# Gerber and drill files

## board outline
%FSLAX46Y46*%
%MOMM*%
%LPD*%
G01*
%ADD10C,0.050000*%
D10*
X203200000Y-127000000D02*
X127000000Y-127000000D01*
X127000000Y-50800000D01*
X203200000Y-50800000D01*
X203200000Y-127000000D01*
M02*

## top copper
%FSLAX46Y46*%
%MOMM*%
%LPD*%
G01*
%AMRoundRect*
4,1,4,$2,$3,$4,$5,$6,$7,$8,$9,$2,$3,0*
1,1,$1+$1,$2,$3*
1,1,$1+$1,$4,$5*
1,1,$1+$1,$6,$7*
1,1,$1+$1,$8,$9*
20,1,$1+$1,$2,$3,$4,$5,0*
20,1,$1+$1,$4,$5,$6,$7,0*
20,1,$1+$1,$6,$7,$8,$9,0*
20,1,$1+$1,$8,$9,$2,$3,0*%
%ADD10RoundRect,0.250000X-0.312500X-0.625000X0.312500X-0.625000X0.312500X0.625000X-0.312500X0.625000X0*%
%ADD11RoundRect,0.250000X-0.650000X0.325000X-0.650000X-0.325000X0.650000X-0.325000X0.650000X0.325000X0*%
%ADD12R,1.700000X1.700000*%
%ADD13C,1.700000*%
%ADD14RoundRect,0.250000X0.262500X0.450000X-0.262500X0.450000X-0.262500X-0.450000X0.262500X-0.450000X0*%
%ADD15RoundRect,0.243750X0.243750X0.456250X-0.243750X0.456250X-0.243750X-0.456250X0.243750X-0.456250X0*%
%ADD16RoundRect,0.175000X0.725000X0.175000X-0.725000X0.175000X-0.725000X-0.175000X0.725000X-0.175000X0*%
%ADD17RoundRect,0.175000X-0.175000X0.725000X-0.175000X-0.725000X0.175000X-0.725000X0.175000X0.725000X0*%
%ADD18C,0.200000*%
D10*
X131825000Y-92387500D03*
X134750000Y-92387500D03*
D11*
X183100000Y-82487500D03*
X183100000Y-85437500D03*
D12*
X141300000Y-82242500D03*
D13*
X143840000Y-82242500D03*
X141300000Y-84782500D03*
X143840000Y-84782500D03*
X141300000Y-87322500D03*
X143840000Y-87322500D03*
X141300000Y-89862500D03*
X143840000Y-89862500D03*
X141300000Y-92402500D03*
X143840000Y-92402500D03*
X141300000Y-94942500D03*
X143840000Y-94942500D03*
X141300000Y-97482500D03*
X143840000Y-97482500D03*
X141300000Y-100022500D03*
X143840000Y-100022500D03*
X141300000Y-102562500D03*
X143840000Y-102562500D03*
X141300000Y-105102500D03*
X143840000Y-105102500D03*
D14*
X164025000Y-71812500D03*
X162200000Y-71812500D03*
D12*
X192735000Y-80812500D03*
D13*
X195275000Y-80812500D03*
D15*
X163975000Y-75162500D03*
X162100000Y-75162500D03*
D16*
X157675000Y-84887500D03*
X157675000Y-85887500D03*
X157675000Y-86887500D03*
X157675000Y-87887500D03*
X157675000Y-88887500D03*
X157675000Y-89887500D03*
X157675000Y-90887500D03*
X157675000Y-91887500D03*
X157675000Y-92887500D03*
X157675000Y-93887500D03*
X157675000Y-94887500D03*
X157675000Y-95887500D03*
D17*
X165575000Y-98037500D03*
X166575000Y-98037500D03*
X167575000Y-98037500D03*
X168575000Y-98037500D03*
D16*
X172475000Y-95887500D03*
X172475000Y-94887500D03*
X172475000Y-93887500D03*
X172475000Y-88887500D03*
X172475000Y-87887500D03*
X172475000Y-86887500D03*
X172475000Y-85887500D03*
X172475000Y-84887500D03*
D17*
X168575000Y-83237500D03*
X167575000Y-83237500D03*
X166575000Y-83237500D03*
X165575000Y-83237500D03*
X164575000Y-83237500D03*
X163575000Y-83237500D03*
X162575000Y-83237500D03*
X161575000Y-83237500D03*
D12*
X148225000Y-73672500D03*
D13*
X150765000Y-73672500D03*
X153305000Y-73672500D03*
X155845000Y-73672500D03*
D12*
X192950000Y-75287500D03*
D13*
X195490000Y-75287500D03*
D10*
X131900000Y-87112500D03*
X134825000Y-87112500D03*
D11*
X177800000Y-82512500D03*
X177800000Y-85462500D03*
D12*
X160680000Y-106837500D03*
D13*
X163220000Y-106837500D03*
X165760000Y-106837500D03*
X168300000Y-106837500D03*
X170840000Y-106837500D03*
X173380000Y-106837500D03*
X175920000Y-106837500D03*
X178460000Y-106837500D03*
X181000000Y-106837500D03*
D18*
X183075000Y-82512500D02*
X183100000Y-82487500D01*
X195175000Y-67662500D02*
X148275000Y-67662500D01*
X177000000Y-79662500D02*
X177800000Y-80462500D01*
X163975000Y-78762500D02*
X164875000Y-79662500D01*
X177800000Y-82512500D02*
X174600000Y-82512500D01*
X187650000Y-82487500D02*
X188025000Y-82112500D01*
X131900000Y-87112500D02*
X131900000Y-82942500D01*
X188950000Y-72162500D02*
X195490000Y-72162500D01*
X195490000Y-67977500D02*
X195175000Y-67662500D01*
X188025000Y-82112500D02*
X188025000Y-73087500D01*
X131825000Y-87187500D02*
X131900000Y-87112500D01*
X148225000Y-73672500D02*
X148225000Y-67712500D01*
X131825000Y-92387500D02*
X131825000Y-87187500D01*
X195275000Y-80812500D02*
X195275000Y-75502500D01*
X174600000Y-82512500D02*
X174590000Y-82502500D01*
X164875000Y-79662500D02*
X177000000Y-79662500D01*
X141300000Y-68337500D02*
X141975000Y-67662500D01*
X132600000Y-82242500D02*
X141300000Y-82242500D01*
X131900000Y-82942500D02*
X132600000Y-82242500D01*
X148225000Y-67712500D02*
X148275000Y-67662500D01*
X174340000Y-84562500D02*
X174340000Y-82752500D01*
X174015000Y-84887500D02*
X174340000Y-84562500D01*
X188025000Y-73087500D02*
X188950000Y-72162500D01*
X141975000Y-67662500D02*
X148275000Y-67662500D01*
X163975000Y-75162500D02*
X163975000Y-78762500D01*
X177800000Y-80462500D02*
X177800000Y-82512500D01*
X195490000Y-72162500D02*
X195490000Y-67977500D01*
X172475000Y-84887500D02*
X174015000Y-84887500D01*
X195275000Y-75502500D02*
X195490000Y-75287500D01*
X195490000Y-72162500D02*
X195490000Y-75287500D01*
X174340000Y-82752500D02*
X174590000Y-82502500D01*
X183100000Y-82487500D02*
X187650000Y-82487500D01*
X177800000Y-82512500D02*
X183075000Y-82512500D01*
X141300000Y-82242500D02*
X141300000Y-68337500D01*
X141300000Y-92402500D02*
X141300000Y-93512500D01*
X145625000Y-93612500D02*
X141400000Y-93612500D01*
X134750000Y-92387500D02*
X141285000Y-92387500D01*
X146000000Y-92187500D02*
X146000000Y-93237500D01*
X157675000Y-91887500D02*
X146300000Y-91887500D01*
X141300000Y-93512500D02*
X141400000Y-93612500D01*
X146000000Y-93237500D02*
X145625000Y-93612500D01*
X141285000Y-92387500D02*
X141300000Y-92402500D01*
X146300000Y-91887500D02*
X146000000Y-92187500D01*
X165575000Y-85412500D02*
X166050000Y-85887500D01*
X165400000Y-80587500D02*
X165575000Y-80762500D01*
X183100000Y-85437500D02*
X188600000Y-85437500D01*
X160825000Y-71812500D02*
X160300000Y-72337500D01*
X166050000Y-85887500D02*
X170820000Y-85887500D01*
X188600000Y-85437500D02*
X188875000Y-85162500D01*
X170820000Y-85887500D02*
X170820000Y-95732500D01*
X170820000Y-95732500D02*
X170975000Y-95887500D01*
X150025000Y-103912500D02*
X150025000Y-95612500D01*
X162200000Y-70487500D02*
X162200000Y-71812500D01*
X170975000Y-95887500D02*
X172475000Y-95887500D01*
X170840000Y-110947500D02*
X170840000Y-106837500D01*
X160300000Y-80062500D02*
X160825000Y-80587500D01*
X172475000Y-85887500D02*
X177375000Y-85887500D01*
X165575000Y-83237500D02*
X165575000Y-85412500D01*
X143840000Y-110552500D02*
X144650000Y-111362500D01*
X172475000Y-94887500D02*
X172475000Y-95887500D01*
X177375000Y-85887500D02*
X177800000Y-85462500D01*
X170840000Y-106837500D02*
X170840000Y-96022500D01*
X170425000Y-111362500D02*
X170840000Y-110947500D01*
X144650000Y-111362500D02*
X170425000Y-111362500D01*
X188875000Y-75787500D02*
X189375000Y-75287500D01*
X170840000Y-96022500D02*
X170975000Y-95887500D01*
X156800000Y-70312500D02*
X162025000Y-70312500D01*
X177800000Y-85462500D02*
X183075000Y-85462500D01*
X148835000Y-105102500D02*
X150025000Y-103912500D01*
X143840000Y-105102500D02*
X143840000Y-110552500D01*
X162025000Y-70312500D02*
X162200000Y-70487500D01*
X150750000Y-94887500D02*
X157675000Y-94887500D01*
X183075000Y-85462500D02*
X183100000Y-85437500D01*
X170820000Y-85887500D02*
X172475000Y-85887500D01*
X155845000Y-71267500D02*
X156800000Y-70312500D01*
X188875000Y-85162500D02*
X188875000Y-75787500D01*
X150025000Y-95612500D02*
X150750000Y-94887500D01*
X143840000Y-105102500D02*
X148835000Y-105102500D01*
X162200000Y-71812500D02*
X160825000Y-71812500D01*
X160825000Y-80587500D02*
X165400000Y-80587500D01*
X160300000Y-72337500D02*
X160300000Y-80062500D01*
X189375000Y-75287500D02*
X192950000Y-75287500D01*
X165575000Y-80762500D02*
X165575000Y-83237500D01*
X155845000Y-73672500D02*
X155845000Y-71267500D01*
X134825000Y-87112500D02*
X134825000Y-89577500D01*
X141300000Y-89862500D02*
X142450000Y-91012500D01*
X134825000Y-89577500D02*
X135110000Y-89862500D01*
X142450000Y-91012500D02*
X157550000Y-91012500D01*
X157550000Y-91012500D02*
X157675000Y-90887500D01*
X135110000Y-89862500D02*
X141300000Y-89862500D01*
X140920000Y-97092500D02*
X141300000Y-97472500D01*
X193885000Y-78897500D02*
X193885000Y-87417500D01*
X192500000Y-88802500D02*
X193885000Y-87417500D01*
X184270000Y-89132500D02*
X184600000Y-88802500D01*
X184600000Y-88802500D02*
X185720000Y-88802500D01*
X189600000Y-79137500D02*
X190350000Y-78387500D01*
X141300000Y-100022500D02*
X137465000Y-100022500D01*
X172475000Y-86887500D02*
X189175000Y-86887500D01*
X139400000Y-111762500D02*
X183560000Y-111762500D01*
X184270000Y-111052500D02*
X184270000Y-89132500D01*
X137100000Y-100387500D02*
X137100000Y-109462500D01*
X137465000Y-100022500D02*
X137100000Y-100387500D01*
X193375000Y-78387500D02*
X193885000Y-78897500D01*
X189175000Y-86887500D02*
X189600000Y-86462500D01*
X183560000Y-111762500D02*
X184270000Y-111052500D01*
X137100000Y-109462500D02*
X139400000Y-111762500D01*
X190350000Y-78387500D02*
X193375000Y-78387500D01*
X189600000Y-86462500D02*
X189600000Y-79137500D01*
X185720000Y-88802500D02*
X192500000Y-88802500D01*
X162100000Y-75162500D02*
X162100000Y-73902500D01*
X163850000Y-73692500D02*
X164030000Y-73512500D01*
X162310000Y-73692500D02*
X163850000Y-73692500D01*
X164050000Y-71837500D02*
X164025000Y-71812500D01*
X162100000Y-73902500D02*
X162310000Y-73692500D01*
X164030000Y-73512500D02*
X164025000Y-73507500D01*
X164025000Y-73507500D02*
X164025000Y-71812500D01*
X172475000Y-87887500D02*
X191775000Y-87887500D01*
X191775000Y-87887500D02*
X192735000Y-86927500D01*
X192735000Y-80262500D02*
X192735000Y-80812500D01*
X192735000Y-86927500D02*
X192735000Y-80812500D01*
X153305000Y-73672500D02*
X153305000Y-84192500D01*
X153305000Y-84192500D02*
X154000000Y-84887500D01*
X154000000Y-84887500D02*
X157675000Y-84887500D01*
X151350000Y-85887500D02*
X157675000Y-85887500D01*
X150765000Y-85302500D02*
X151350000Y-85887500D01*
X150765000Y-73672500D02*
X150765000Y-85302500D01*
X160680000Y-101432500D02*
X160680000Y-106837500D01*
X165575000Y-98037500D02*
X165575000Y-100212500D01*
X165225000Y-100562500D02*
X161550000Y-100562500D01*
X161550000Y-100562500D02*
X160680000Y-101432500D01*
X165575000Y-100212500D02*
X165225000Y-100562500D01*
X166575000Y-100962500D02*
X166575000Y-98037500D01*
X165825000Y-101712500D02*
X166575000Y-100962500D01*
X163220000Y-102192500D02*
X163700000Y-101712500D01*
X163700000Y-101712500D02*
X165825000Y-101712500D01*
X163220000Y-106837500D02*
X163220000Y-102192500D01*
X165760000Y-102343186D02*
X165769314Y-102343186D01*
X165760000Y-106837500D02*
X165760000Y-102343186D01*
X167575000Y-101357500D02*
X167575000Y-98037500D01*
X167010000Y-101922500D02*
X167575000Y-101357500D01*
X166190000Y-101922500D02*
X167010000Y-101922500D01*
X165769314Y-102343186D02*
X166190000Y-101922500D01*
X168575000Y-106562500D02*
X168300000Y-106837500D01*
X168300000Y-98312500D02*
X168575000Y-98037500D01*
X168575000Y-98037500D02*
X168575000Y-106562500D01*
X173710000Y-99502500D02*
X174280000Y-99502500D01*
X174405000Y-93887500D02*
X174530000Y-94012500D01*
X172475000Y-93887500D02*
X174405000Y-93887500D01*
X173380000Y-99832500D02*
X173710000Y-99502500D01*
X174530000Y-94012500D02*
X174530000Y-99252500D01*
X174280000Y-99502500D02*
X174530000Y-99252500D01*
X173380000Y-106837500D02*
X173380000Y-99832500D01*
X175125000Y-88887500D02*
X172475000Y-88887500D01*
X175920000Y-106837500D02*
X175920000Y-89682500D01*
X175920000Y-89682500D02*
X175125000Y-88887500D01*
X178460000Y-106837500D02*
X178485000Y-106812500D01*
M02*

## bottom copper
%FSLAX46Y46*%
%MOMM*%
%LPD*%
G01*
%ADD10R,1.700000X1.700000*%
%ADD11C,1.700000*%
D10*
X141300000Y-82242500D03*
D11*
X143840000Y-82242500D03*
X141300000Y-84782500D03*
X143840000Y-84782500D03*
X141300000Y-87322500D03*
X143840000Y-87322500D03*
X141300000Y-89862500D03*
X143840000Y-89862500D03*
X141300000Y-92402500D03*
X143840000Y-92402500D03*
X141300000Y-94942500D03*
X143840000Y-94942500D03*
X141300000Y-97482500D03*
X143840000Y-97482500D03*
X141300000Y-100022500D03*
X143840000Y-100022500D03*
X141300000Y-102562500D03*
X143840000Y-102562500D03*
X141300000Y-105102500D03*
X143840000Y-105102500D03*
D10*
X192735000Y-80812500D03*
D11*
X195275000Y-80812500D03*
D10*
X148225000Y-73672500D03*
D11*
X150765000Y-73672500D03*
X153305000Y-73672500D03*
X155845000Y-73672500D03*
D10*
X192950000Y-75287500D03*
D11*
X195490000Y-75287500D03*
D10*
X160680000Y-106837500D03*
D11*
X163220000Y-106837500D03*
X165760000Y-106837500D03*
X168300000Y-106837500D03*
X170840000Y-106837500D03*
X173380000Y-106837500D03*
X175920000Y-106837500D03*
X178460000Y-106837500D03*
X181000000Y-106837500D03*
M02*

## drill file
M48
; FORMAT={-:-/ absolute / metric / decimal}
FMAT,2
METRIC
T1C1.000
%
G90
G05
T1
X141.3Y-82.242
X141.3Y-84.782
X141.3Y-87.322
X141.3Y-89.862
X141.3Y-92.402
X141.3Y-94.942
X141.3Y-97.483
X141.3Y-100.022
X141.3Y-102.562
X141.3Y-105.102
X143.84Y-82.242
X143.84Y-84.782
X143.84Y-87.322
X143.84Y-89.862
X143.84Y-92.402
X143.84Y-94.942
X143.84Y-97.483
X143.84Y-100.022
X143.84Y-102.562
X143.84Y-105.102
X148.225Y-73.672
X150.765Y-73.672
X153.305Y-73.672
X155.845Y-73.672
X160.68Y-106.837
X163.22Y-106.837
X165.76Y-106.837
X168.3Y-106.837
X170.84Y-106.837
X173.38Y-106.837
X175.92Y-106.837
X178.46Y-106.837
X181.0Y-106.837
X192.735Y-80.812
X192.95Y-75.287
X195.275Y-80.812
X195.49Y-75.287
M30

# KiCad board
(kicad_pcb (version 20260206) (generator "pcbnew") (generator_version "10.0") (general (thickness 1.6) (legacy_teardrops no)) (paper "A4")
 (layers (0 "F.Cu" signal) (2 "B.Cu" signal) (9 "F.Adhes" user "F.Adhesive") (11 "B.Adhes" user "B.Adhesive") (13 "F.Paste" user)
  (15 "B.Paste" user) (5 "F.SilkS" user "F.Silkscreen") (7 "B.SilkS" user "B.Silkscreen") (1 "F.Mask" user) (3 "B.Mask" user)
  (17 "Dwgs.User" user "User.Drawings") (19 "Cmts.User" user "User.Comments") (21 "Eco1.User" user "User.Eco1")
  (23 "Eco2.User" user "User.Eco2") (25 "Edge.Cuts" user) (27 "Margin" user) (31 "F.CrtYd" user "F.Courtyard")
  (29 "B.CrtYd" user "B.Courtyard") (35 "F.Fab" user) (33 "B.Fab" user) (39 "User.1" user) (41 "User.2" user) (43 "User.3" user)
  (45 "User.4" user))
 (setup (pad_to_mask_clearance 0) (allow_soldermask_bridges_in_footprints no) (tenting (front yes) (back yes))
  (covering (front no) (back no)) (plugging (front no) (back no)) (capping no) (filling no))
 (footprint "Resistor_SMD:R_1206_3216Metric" (layer "F.Cu") (at 133.2875 92.3875)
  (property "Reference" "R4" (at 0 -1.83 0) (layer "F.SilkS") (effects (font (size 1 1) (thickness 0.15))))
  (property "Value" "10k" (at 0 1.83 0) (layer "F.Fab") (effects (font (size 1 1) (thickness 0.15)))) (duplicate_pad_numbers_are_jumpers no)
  (pad "1" smd roundrect (at -1.4625 0) (size 1.125 1.75) (layers "F.Cu" "F.Mask" "F.Paste") (roundrect_rratio 0.222222) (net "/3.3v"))
  (pad "2" smd roundrect (at 1.4625 0) (size 1.125 1.75) (layers "F.Cu" "F.Mask" "F.Paste") (roundrect_rratio 0.222222) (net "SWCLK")))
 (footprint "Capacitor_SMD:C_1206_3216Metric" (layer "F.Cu") (at 183.1 83.9625 -90)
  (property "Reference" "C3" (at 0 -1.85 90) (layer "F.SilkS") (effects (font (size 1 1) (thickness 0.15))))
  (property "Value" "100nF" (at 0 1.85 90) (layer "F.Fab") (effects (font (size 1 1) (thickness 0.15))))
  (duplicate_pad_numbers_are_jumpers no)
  (pad "1" smd roundrect (at -1.475 0 270) (size 1.15 1.8) (layers "F.Cu" "F.Mask" "F.Paste") (roundrect_rratio 0.217391) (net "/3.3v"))
  (pad "2" smd roundrect (at 1.475 0 270) (size 1.15 1.8) (layers "F.Cu" "F.Mask" "F.Paste") (roundrect_rratio 0.217391) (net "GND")))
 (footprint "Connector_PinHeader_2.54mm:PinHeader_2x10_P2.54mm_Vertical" (layer "F.Cu") (at 141.3 82.2425)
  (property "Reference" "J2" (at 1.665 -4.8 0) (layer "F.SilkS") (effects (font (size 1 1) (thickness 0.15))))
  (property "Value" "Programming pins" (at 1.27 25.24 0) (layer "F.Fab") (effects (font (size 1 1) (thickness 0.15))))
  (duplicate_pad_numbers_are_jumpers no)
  (pad "1" thru_hole rect (at 0 0) (size 1.7 1.7) (drill 1) (layers "*.Cu" "*.Mask") (remove_unused_layers no) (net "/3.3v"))
  (pad "2" thru_hole circle (at 2.54 0) (size 1.7 1.7) (drill 1) (layers "*.Cu" "*.Mask") (remove_unused_layers no)
   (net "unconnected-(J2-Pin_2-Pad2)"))
  (pad "3" thru_hole circle (at 0 2.54) (size 1.7 1.7) (drill 1) (layers "*.Cu" "*.Mask") (remove_unused_layers no)
   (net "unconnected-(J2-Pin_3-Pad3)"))
  (pad "4" thru_hole circle (at 2.54 2.54) (size 1.7 1.7) (drill 1) (layers "*.Cu" "*.Mask") (remove_unused_layers no)
   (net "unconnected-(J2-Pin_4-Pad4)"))
  (pad "5" thru_hole circle (at 0 5.08) (size 1.7 1.7) (drill 1) (layers "*.Cu" "*.Mask") (remove_unused_layers no)
   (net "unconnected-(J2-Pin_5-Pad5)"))
  (pad "6" thru_hole circle (at 2.54 5.08) (size 1.7 1.7) (drill 1) (layers "*.Cu" "*.Mask") (remove_unused_layers no)
   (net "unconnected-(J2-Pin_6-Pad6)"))
  (pad "7" thru_hole circle (at 0 7.62) (size 1.7 1.7) (drill 1) (layers "*.Cu" "*.Mask") (remove_unused_layers no) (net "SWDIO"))
  (pad "8" thru_hole circle (at 2.54 7.62) (size 1.7 1.7) (drill 1) (layers "*.Cu" "*.Mask") (remove_unused_layers no)
   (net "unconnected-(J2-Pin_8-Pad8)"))
  (pad "9" thru_hole circle (at 0 10.16) (size 1.7 1.7) (drill 1) (layers "*.Cu" "*.Mask") (remove_unused_layers no) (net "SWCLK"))
  (pad "10" thru_hole circle (at 2.54 10.16) (size 1.7 1.7) (drill 1) (layers "*.Cu" "*.Mask") (remove_unused_layers no)
   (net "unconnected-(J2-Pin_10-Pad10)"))
  (pad "11" thru_hole circle (at 0 12.7) (size 1.7 1.7) (drill 1) (layers "*.Cu" "*.Mask") (remove_unused_layers no)
   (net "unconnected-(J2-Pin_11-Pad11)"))
  (pad "12" thru_hole circle (at 2.54 12.7) (size 1.7 1.7) (drill 1) (layers "*.Cu" "*.Mask") (remove_unused_layers no)
   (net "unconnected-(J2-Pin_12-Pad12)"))
  (pad "13" thru_hole circle (at 0 15.24) (size 1.7 1.7) (drill 1) (layers "*.Cu" "*.Mask") (remove_unused_layers no)
   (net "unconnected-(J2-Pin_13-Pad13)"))
  (pad "14" thru_hole circle (at 2.54 15.24) (size 1.7 1.7) (drill 1) (layers "*.Cu" "*.Mask") (remove_unused_layers no)
   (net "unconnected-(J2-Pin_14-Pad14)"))
  (pad "15" thru_hole circle (at 0 17.78) (size 1.7 1.7) (drill 1) (layers "*.Cu" "*.Mask") (remove_unused_layers no) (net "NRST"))
  (pad "16" thru_hole circle (at 2.54 17.78) (size 1.7 1.7) (drill 1) (layers "*.Cu" "*.Mask") (remove_unused_layers no)
   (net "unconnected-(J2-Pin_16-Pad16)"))
  (pad "17" thru_hole circle (at 0 20.32) (size 1.7 1.7) (drill 1) (layers "*.Cu" "*.Mask") (remove_unused_layers no)
   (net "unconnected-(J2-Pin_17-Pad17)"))
  (pad "18" thru_hole circle (at 2.54 20.32) (size 1.7 1.7) (drill 1) (layers "*.Cu" "*.Mask") (remove_unused_layers no)
   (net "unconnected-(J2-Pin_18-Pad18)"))
  (pad "19" thru_hole circle (at 0 22.86) (size 1.7 1.7) (drill 1) (layers "*.Cu" "*.Mask") (remove_unused_layers no)
   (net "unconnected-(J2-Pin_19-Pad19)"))
  (pad "20" thru_hole circle (at 2.54 22.86) (size 1.7 1.7) (drill 1) (layers "*.Cu" "*.Mask") (remove_unused_layers no) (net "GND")))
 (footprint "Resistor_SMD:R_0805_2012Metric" (layer "F.Cu") (at 163.1125 71.8125 180)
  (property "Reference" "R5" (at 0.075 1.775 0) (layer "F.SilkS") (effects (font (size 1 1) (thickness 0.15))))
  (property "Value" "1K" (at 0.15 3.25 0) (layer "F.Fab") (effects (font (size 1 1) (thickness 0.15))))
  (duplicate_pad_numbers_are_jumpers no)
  (pad "1" smd roundrect (at -0.9125 0 180) (size 1.025 1.4) (layers "F.Cu" "F.Mask" "F.Paste") (roundrect_rratio 0.243902)
   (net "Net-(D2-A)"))
  (pad "2" smd roundrect (at 0.9125 0 180) (size 1.025 1.4) (layers "F.Cu" "F.Mask" "F.Paste") (roundrect_rratio 0.243902) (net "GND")))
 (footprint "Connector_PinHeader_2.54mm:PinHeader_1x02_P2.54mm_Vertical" (layer "F.Cu") (at 192.735 80.8125 90)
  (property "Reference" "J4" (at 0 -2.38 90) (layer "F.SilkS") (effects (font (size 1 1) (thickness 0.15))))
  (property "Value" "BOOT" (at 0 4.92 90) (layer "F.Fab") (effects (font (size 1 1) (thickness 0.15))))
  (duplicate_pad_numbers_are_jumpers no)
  (pad "1" thru_hole rect (at 0 0 90) (size 1.7 1.7) (drill 1) (layers "*.Cu" "*.Mask") (remove_unused_layers no) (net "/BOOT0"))
  (pad "2" thru_hole circle (at 0 2.54 90) (size 1.7 1.7) (drill 1) (layers "*.Cu" "*.Mask") (remove_unused_layers no) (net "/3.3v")))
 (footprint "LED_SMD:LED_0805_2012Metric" (layer "F.Cu") (at 163.0375 75.1625 180)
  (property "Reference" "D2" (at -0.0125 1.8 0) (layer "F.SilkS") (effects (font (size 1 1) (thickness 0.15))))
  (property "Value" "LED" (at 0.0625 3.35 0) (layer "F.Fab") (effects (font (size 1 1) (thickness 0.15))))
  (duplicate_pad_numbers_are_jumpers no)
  (pad "1" smd roundrect (at -0.9375 0 180) (size 0.975 1.4) (layers "F.Cu" "F.Mask" "F.Paste") (roundrect_rratio 0.25) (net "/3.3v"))
  (pad "2" smd roundrect (at 0.9375 0 180) (size 0.975 1.4) (layers "F.Cu" "F.Mask" "F.Paste") (roundrect_rratio 0.25) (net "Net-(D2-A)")))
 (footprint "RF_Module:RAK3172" (layer "F.Cu") (at 165.075 90.6375)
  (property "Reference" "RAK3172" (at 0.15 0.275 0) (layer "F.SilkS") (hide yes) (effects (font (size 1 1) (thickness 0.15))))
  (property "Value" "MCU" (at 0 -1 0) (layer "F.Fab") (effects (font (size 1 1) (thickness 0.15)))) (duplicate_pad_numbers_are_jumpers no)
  (pad "1" smd roundrect (at -7.4 -5.75 180) (size 1.8 0.7) (layers "F.Cu" "F.Mask" "F.Paste") (roundrect_rratio 0.25) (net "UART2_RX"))
  (pad "2" smd roundrect (at -7.4 -4.75 180) (size 1.8 0.7) (layers "F.Cu" "F.Mask" "F.Paste") (roundrect_rratio 0.25) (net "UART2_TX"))
  (pad "3" smd roundrect (at -7.4 -3.75 180) (size 1.8 0.7) (layers "F.Cu" "F.Mask" "F.Paste") (roundrect_rratio 0.25)
   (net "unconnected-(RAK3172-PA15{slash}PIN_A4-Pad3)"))
  (pad "4" smd roundrect (at -7.4 -2.75 180) (size 1.8 0.7) (layers "F.Cu" "F.Mask" "F.Paste") (roundrect_rratio 0.25)
   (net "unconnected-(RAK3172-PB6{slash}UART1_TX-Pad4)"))
  (pad "5" smd roundrect (at -7.4 -1.75 180) (size 1.8 0.7) (layers "F.Cu" "F.Mask" "F.Paste") (roundrect_rratio 0.25)
   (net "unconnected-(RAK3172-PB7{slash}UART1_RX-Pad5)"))
  (pad "6" smd roundrect (at -7.4 -0.75 180) (size 1.8 0.7) (layers "F.Cu" "F.Mask" "F.Paste") (roundrect_rratio 0.25)
   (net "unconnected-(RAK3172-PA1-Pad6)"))
  (pad "7" smd roundrect (at -7.4 0.25 180) (size 1.8 0.7) (layers "F.Cu" "F.Mask" "F.Paste") (roundrect_rratio 0.25) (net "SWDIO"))
  (pad "8" smd roundrect (at -7.4 1.25 180) (size 1.8 0.7) (layers "F.Cu" "F.Mask" "F.Paste") (roundrect_rratio 0.25) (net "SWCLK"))
  (pad "9" smd roundrect (at -7.4 2.25 180) (size 1.8 0.7) (layers "F.Cu" "F.Mask" "F.Paste") (roundrect_rratio 0.25)
   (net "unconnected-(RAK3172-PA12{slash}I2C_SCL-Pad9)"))
  (pad "10" smd roundrect (at -7.4 3.25 180) (size 1.8 0.7) (layers "F.Cu" "F.Mask" "F.Paste") (roundrect_rratio 0.25)
   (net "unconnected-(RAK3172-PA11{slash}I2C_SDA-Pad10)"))
  (pad "11" smd roundrect (at -7.4 4.25 180) (size 1.8 0.7) (layers "F.Cu" "F.Mask" "F.Paste") (roundrect_rratio 0.25) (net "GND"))
  (pad "12" smd roundrect (at -7.4 5.25 180) (size 1.8 0.7) (layers "F.Cu" "F.Mask" "F.Paste") (roundrect_rratio 0.25)
   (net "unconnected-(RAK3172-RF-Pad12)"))
  (pad "13" smd roundrect (at 0.5 7.4 270) (size 1.8 0.7) (layers "F.Cu" "F.Mask" "F.Paste") (roundrect_rratio 0.25) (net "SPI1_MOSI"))
  (pad "14" smd roundrect (at 1.5 7.4 270) (size 1.8 0.7) (layers "F.Cu" "F.Mask" "F.Paste") (roundrect_rratio 0.25) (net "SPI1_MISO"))
  (pad "15" smd roundrect (at 2.5 7.4 270) (size 1.8 0.7) (layers "F.Cu" "F.Mask" "F.Paste") (roundrect_rratio 0.25) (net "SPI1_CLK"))
  (pad "16" smd roundrect (at 3.5 7.4 270) (size 1.8 0.7) (layers "F.Cu" "F.Mask" "F.Paste") (roundrect_rratio 0.25) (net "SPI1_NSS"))
  (pad "17" smd roundrect (at 7.4 5.25 180) (size 1.8 0.7) (layers "F.Cu" "F.Mask" "F.Paste") (roundrect_rratio 0.25) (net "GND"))
  (pad "18" smd roundrect (at 7.4 4.25 180) (size 1.8 0.7) (layers "F.Cu" "F.Mask" "F.Paste") (roundrect_rratio 0.25) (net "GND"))
  (pad "19" smd roundrect (at 7.4 3.25 180) (size 1.8 0.7) (layers "F.Cu" "F.Mask" "F.Paste") (roundrect_rratio 0.25) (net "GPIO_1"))
  (pad "20" smd roundrect (at 7.4 -1.75 180) (size 1.8 0.7) (layers "F.Cu" "F.Mask" "F.Paste") (roundrect_rratio 0.25) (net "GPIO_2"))
  (pad "21" smd roundrect (at 7.4 -2.75 180) (size 1.8 0.7) (layers "F.Cu" "F.Mask" "F.Paste") (roundrect_rratio 0.25) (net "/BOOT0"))
  (pad "22" smd roundrect (at 7.4 -3.75 180) (size 1.8 0.7) (layers "F.Cu" "F.Mask" "F.Paste") (roundrect_rratio 0.25) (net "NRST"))
  (pad "23" smd roundrect (at 7.4 -4.75 180) (size 1.8 0.7) (layers "F.Cu" "F.Mask" "F.Paste") (roundrect_rratio 0.25) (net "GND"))
  (pad "24" smd roundrect (at 7.4 -5.75 180) (size 1.8 0.7) (layers "F.Cu" "F.Mask" "F.Paste") (roundrect_rratio 0.25) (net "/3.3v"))
  (pad "25" smd roundrect (at 3.5 -7.4 270) (size 1.8 0.7) (layers "F.Cu" "F.Mask" "F.Paste") (roundrect_rratio 0.25)
   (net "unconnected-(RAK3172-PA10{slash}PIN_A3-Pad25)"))
  (pad "26" smd roundrect (at 2.5 -7.4 270) (size 1.8 0.7) (layers "F.Cu" "F.Mask" "F.Paste") (roundrect_rratio 0.25)
   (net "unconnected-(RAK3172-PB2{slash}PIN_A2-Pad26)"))
  (pad "27" smd roundrect (at 1.5 -7.4 270) (size 1.8 0.7) (layers "F.Cu" "F.Mask" "F.Paste") (roundrect_rratio 0.25)
   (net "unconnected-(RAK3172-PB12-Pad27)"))
  (pad "28" smd roundrect (at 0.5 -7.4 270) (size 1.8 0.7) (layers "F.Cu" "F.Mask" "F.Paste") (roundrect_rratio 0.25) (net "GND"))
  (pad "29" smd roundrect (at -0.5 -7.4 270) (size 1.8 0.7) (layers "F.Cu" "F.Mask" "F.Paste") (roundrect_rratio 0.25)
   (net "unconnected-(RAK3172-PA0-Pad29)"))
  (pad "30" smd roundrect (at -1.5 -7.4 270) (size 1.8 0.7) (layers "F.Cu" "F.Mask" "F.Paste") (roundrect_rratio 0.25)
   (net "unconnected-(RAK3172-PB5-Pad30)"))
  (pad "31" smd roundrect (at -2.5 -7.4 270) (size 1.8 0.7) (layers "F.Cu" "F.Mask" "F.Paste") (roundrect_rratio 0.25)
   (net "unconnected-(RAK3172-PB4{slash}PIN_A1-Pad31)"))
  (pad "32" smd roundrect (at -3.5 -7.4 270) (size 1.8 0.7) (layers "F.Cu" "F.Mask" "F.Paste") (roundrect_rratio 0.25)
   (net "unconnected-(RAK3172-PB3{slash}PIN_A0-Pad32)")))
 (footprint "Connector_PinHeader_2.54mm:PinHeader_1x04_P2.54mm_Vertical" (layer "F.Cu") (at 148.225 73.6725 90)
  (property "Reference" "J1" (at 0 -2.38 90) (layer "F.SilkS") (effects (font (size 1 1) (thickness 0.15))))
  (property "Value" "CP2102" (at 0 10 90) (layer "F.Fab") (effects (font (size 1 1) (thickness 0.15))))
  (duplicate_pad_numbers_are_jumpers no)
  (pad "1" thru_hole rect (at 0 0 90) (size 1.7 1.7) (drill 1) (layers "*.Cu" "*.Mask") (remove_unused_layers no) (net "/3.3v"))
  (pad "2" thru_hole circle (at 0 2.54 90) (size 1.7 1.7) (drill 1) (layers "*.Cu" "*.Mask") (remove_unused_layers no) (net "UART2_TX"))
  (pad "3" thru_hole circle (at 0 5.08 90) (size 1.7 1.7) (drill 1) (layers "*.Cu" "*.Mask") (remove_unused_layers no) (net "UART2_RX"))
  (pad "4" thru_hole circle (at 0 7.62 90) (size 1.7 1.7) (drill 1) (layers "*.Cu" "*.Mask") (remove_unused_layers no) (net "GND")))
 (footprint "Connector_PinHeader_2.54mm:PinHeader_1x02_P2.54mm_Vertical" (layer "F.Cu") (at 192.95 75.2875 90)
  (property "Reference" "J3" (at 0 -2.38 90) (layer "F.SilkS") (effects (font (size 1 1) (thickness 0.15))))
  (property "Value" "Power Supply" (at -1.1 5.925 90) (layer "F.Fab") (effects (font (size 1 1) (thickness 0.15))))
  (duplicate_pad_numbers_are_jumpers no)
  (pad "1" thru_hole rect (at 0 0 90) (size 1.7 1.7) (drill 1) (layers "*.Cu" "*.Mask") (remove_unused_layers no) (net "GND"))
  (pad "2" thru_hole circle (at 0 2.54 90) (size 1.7 1.7) (drill 1) (layers "*.Cu" "*.Mask") (remove_unused_layers no) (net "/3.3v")))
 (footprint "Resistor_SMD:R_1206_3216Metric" (layer "F.Cu") (at 133.3625 87.1125)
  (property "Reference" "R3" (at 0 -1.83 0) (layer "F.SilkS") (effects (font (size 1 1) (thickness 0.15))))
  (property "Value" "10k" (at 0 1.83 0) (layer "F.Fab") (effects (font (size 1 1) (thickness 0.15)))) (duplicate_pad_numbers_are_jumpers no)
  (pad "1" smd roundrect (at -1.4625 0) (size 1.125 1.75) (layers "F.Cu" "F.Mask" "F.Paste") (roundrect_rratio 0.222222) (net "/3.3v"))
  (pad "2" smd roundrect (at 1.4625 0) (size 1.125 1.75) (layers "F.Cu" "F.Mask" "F.Paste") (roundrect_rratio 0.222222) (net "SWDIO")))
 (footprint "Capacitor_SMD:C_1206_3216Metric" (layer "F.Cu") (at 177.8 83.9875 -90)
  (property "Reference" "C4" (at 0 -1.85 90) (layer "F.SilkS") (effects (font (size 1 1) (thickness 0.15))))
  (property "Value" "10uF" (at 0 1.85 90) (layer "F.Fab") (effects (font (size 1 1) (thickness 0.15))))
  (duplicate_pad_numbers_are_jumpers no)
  (pad "1" smd roundrect (at -1.475 0 270) (size 1.15 1.8) (layers "F.Cu" "F.Mask" "F.Paste") (roundrect_rratio 0.217391) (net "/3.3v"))
  (pad "2" smd roundrect (at 1.475 0 270) (size 1.15 1.8) (layers "F.Cu" "F.Mask" "F.Paste") (roundrect_rratio 0.217391) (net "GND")))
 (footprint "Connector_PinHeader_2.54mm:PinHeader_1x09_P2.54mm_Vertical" (layer "F.Cu") (at 160.68 106.8375 90)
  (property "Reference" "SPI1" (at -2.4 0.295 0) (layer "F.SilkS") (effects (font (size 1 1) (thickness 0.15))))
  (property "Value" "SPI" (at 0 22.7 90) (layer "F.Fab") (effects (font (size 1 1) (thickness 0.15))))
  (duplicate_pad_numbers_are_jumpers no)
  (pad "1" thru_hole rect (at 0 0 90) (size 1.7 1.7) (drill 1) (layers "*.Cu" "*.Mask") (remove_unused_layers no) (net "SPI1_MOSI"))
  (pad "2" thru_hole circle (at 0 2.54 90) (size 1.7 1.7) (drill 1) (layers "*.Cu" "*.Mask") (remove_unused_layers no) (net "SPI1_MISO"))
  (pad "3" thru_hole circle (at 0 5.08 90) (size 1.7 1.7) (drill 1) (layers "*.Cu" "*.Mask") (remove_unused_layers no) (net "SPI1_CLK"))
  (pad "4" thru_hole circle (at 0 7.62 90) (size 1.7 1.7) (drill 1) (layers "*.Cu" "*.Mask") (remove_unused_layers no) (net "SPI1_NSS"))
  (pad "5" thru_hole circle (at 0 10.16 90) (size 1.7 1.7) (drill 1) (layers "*.Cu" "*.Mask") (remove_unused_layers no) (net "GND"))
  (pad "6" thru_hole circle (at 0 12.7 90) (size 1.7 1.7) (drill 1) (layers "*.Cu" "*.Mask") (remove_unused_layers no) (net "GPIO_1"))
  (pad "7" thru_hole circle (at 0 15.24 90) (size 1.7 1.7) (drill 1) (layers "*.Cu" "*.Mask") (remove_unused_layers no) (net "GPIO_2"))
  (pad "8" thru_hole circle (at 0 17.78 90) (size 1.7 1.7) (drill 1) (layers "*.Cu" "*.Mask") (remove_unused_layers no)
   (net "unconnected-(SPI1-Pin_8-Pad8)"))
  (pad "9" thru_hole circle (at 0 20.32 90) (size 1.7 1.7) (drill 1) (layers "*.Cu" "*.Mask") (remove_unused_layers no)
   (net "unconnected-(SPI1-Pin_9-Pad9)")))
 (gr_poly (pts (xy 203.2 127) (xy 127 127) (xy 127 50.8) (xy 203.2 50.8)) (stroke (width 0.05) (type solid)) (fill no) (layer "Edge.Cuts"))
 (segment (start 183.075 82.5125) (end 183.1 82.4875) (width 0.2) (layer "F.Cu") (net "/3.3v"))
 (segment (start 195.175 67.6625) (end 148.275 67.6625) (width 0.2) (layer "F.Cu") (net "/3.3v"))
 (segment (start 177 79.6625) (end 177.8 80.4625) (width 0.2) (layer "F.Cu") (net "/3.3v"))
 (segment (start 163.975 78.7625) (end 164.875 79.6625) (width 0.2) (layer "F.Cu") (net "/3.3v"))
 (segment (start 177.8 82.5125) (end 174.6 82.5125) (width 0.2) (layer "F.Cu") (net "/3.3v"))
 (segment (start 187.65 82.4875) (end 188.025 82.1125) (width 0.2) (layer "F.Cu") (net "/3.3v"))
 (segment (start 131.9 87.1125) (end 131.9 82.9425) (width 0.2) (layer "F.Cu") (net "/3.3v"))
 (segment (start 188.95 72.1625) (end 195.49 72.1625) (width 0.2) (layer "F.Cu") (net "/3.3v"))
 (segment (start 195.49 67.9775) (end 195.175 67.6625) (width 0.2) (layer "F.Cu") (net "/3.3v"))
 (segment (start 188.025 82.1125) (end 188.025 73.0875) (width 0.2) (layer "F.Cu") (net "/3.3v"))
 (segment (start 131.825 87.1875) (end 131.9 87.1125) (width 0.2) (layer "F.Cu") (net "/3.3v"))
 (segment (start 148.225 73.6725) (end 148.225 67.7125) (width 0.2) (layer "F.Cu") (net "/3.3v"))
 (segment (start 131.825 92.3875) (end 131.825 87.1875) (width 0.2) (layer "F.Cu") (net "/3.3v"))
 (segment (start 195.275 80.8125) (end 195.275 75.5025) (width 0.2) (layer "F.Cu") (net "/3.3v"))
 (segment (start 174.6 82.5125) (end 174.59 82.5025) (width 0.2) (layer "F.Cu") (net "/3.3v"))
 (segment (start 164.875 79.6625) (end 177 79.6625) (width 0.2) (layer "F.Cu") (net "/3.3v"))
 (segment (start 141.3 68.3375) (end 141.975 67.6625) (width 0.2) (layer "F.Cu") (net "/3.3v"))
 (segment (start 132.6 82.2425) (end 141.3 82.2425) (width 0.2) (layer "F.Cu") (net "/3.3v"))
 (segment (start 131.9 82.9425) (end 132.6 82.2425) (width 0.2) (layer "F.Cu") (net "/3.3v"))
 (segment (start 148.225 67.7125) (end 148.275 67.6625) (width 0.2) (layer "F.Cu") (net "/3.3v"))
 (segment (start 174.34 84.5625) (end 174.34 82.7525) (width 0.2) (layer "F.Cu") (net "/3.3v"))
 (segment (start 174.015 84.8875) (end 174.34 84.5625) (width 0.2) (layer "F.Cu") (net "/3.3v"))
 (segment (start 188.025 73.0875) (end 188.95 72.1625) (width 0.2) (layer "F.Cu") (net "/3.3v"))
 (segment (start 141.975 67.6625) (end 148.275 67.6625) (width 0.2) (layer "F.Cu") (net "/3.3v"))
 (segment (start 163.975 75.1625) (end 163.975 78.7625) (width 0.2) (layer "F.Cu") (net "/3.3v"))
 (segment (start 177.8 80.4625) (end 177.8 82.5125) (width 0.2) (layer "F.Cu") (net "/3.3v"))
 (segment (start 195.49 72.1625) (end 195.49 67.9775) (width 0.2) (layer "F.Cu") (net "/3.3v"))
 (segment (start 172.475 84.8875) (end 174.015 84.8875) (width 0.2) (layer "F.Cu") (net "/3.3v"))
 (segment (start 195.275 75.5025) (end 195.49 75.2875) (width 0.2) (layer "F.Cu") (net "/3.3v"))
 (segment (start 195.49 72.1625) (end 195.49 75.2875) (width 0.2) (layer "F.Cu") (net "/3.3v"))
 (segment (start 174.34 82.7525) (end 174.59 82.5025) (width 0.2) (layer "F.Cu") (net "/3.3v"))
 (segment (start 183.1 82.4875) (end 187.65 82.4875) (width 0.2) (layer "F.Cu") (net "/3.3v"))
 (segment (start 177.8 82.5125) (end 183.075 82.5125) (width 0.2) (layer "F.Cu") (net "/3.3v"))
 (segment (start 141.3 82.2425) (end 141.3 68.3375) (width 0.2) (layer "F.Cu") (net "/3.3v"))
 (segment (start 141.3 92.4025) (end 141.3 93.5125) (width 0.2) (layer "F.Cu") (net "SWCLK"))
 (segment (start 145.625 93.6125) (end 141.4 93.6125) (width 0.2) (layer "F.Cu") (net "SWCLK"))
 (segment (start 134.75 92.3875) (end 141.285 92.3875) (width 0.2) (layer "F.Cu") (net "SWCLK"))
 (segment (start 146 92.1875) (end 146 93.2375) (width 0.2) (layer "F.Cu") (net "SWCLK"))
 (segment (start 157.675 91.8875) (end 146.3 91.8875) (width 0.2) (layer "F.Cu") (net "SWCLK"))
 (segment (start 141.3 93.5125) (end 141.4 93.6125) (width 0.2) (layer "F.Cu") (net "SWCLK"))
 (segment (start 146 93.2375) (end 145.625 93.6125) (width 0.2) (layer "F.Cu") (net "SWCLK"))
 (segment (start 141.285 92.3875) (end 141.3 92.4025) (width 0.2) (layer "F.Cu") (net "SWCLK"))
 (segment (start 146.3 91.8875) (end 146 92.1875) (width 0.2) (layer "F.Cu") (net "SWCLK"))
 (segment (start 165.575 85.4125) (end 166.05 85.8875) (width 0.2) (layer "F.Cu") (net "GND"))
 (segment (start 165.4 80.5875) (end 165.575 80.7625) (width 0.2) (layer "F.Cu") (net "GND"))
 (segment (start 183.1 85.4375) (end 188.6 85.4375) (width 0.2) (layer "F.Cu") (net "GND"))
 (segment (start 160.825 71.8125) (end 160.3 72.3375) (width 0.2) (layer "F.Cu") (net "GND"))
 (segment (start 166.05 85.8875) (end 170.82 85.8875) (width 0.2) (layer "F.Cu") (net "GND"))
 (segment (start 188.6 85.4375) (end 188.875 85.1625) (width 0.2) (layer "F.Cu") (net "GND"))
 (segment (start 170.82 85.8875) (end 170.82 95.7325) (width 0.2) (layer "F.Cu") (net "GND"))
 (segment (start 170.82 95.7325) (end 170.975 95.8875) (width 0.2) (layer "F.Cu") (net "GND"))
 (segment (start 150.025 103.9125) (end 150.025 95.6125) (width 0.2) (layer "F.Cu") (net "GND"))
 (segment (start 162.2 70.4875) (end 162.2 71.8125) (width 0.2) (layer "F.Cu") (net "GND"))
 (segment (start 170.975 95.8875) (end 172.475 95.8875) (width 0.2) (layer "F.Cu") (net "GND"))
 (segment (start 170.84 110.9475) (end 170.84 106.8375) (width 0.2) (layer "F.Cu") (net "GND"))
 (segment (start 160.3 80.0625) (end 160.825 80.5875) (width 0.2) (layer "F.Cu") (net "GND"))
 (segment (start 172.475 85.8875) (end 177.375 85.8875) (width 0.2) (layer "F.Cu") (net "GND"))
 (segment (start 165.575 83.2375) (end 165.575 85.4125) (width 0.2) (layer "F.Cu") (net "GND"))
 (segment (start 143.84 110.5525) (end 144.65 111.3625) (width 0.2) (layer "F.Cu") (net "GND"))
 (segment (start 172.475 94.8875) (end 172.475 95.8875) (width 0.2) (layer "F.Cu") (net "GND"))
 (segment (start 177.375 85.8875) (end 177.8 85.4625) (width 0.2) (layer "F.Cu") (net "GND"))
 (segment (start 170.84 106.8375) (end 170.84 96.0225) (width 0.2) (layer "F.Cu") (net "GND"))
 (segment (start 170.425 111.3625) (end 170.84 110.9475) (width 0.2) (layer "F.Cu") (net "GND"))
 (segment (start 144.65 111.3625) (end 170.425 111.3625) (width 0.2) (layer "F.Cu") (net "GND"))
 (segment (start 188.875 75.7875) (end 189.375 75.2875) (width 0.2) (layer "F.Cu") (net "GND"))
 (segment (start 170.84 96.0225) (end 170.975 95.8875) (width 0.2) (layer "F.Cu") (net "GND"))
 (segment (start 156.8 70.3125) (end 162.025 70.3125) (width 0.2) (layer "F.Cu") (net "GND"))
 (segment (start 177.8 85.4625) (end 183.075 85.4625) (width 0.2) (layer "F.Cu") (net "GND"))
 (segment (start 148.835 105.1025) (end 150.025 103.9125) (width 0.2) (layer "F.Cu") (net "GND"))
 (segment (start 143.84 105.1025) (end 143.84 110.5525) (width 0.2) (layer "F.Cu") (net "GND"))
 (segment (start 162.025 70.3125) (end 162.2 70.4875) (width 0.2) (layer "F.Cu") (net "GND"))
 (segment (start 150.75 94.8875) (end 157.675 94.8875) (width 0.2) (layer "F.Cu") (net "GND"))
 (segment (start 183.075 85.4625) (end 183.1 85.4375) (width 0.2) (layer "F.Cu") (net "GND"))
 (segment (start 170.82 85.8875) (end 172.475 85.8875) (width 0.2) (layer "F.Cu") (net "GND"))
 (segment (start 155.845 71.2675) (end 156.8 70.3125) (width 0.2) (layer "F.Cu") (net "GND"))
 (segment (start 188.875 85.1625) (end 188.875 75.7875) (width 0.2) (layer "F.Cu") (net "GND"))
 (segment (start 150.025 95.6125) (end 150.75 94.8875) (width 0.2) (layer "F.Cu") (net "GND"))
 (segment (start 143.84 105.1025) (end 148.835 105.1025) (width 0.2) (layer "F.Cu") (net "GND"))
 (segment (start 162.2 71.8125) (end 160.825 71.8125) (width 0.2) (layer "F.Cu") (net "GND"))
 (segment (start 160.825 80.5875) (end 165.4 80.5875) (width 0.2) (layer "F.Cu") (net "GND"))
 (segment (start 160.3 72.3375) (end 160.3 80.0625) (width 0.2) (layer "F.Cu") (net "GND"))
 (segment (start 189.375 75.2875) (end 192.95 75.2875) (width 0.2) (layer "F.Cu") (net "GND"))
 (segment (start 165.575 80.7625) (end 165.575 83.2375) (width 0.2) (layer "F.Cu") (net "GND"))
 (segment (start 155.845 73.6725) (end 155.845 71.2675) (width 0.2) (layer "F.Cu") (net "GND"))
 (segment (start 134.825 87.1125) (end 134.825 89.5775) (width 0.2) (layer "F.Cu") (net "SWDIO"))
 (segment (start 141.3 89.8625) (end 142.45 91.0125) (width 0.2) (layer "F.Cu") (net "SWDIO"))
 (segment (start 134.825 89.5775) (end 135.11 89.8625) (width 0.2) (layer "F.Cu") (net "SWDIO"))
 (segment (start 142.45 91.0125) (end 157.55 91.0125) (width 0.2) (layer "F.Cu") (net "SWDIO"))
 (segment (start 157.55 91.0125) (end 157.675 90.8875) (width 0.2) (layer "F.Cu") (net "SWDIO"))
 (segment (start 135.11 89.8625) (end 141.3 89.8625) (width 0.2) (layer "F.Cu") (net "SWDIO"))
 (segment (start 140.92 97.0925) (end 141.3 97.4725) (width 0.2) (layer "F.Cu") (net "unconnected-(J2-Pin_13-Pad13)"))
 (segment (start 193.885 78.8975) (end 193.885 87.4175) (width 0.2) (layer "F.Cu") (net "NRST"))
 (segment (start 192.5 88.8025) (end 193.885 87.4175) (width 0.2) (layer "F.Cu") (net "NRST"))
 (segment (start 184.27 89.1325) (end 184.6 88.8025) (width 0.2) (layer "F.Cu") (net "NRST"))
 (segment (start 184.6 88.8025) (end 185.72 88.8025) (width 0.2) (layer "F.Cu") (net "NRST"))
 (segment (start 189.6 79.1375) (end 190.35 78.3875) (width 0.2) (layer "F.Cu") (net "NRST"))
 (segment (start 141.3 100.0225) (end 137.465 100.0225) (width 0.2) (layer "F.Cu") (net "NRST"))
 (segment (start 172.475 86.8875) (end 189.175 86.8875) (width 0.2) (layer "F.Cu") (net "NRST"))
 (segment (start 139.4 111.7625) (end 183.56 111.7625) (width 0.2) (layer "F.Cu") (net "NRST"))
 (segment (start 184.27 111.0525) (end 184.27 89.1325) (width 0.2) (layer "F.Cu") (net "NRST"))
 (segment (start 137.1 100.3875) (end 137.1 109.4625) (width 0.2) (layer "F.Cu") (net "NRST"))
 (segment (start 137.465 100.0225) (end 137.1 100.3875) (width 0.2) (layer "F.Cu") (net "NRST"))
 (segment (start 193.375 78.3875) (end 193.885 78.8975) (width 0.2) (layer "F.Cu") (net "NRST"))
 (segment (start 189.175 86.8875) (end 189.6 86.4625) (width 0.2) (layer "F.Cu") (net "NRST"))
 (segment (start 183.56 111.7625) (end 184.27 111.0525) (width 0.2) (layer "F.Cu") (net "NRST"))
 (segment (start 137.1 109.4625) (end 139.4 111.7625) (width 0.2) (layer "F.Cu") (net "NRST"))
 (segment (start 190.35 78.3875) (end 193.375 78.3875) (width 0.2) (layer "F.Cu") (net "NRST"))
 (segment (start 189.6 86.4625) (end 189.6 79.1375) (width 0.2) (layer "F.Cu") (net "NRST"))
 (segment (start 185.72 88.8025) (end 192.5 88.8025) (width 0.2) (layer "F.Cu") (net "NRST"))
 (segment (start 162.1 75.1625) (end 162.1 73.9025) (width 0.2) (layer "F.Cu") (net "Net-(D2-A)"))
 (segment (start 163.85 73.6925) (end 164.03 73.5125) (width 0.2) (layer "F.Cu") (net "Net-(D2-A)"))
 (segment (start 162.31 73.6925) (end 163.85 73.6925) (width 0.2) (layer "F.Cu") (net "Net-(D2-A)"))
 (segment (start 164.05 71.8375) (end 164.025 71.8125) (width 0.2) (layer "F.Cu") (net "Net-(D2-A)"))
 (segment (start 162.1 73.9025) (end 162.31 73.6925) (width 0.2) (layer "F.Cu") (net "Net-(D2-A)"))
 (segment (start 164.03 73.5125) (end 164.025 73.5075) (width 0.2) (layer "F.Cu") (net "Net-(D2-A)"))
 (segment (start 164.025 73.5075) (end 164.025 71.8125) (width 0.2) (layer "F.Cu") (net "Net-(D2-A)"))
 (segment (start 172.475 87.8875) (end 191.775 87.8875) (width 0.2) (layer "F.Cu") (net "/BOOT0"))
 (segment (start 191.775 87.8875) (end 192.735 86.9275) (width 0.2) (layer "F.Cu") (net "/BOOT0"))
 (segment (start 192.735 80.2625) (end 192.735 80.8125) (width 0.2) (layer "F.Cu") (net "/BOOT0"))
 (segment (start 192.735 86.9275) (end 192.735 80.8125) (width 0.2) (layer "F.Cu") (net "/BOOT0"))
 (segment (start 153.305 73.6725) (end 153.305 84.1925) (width 0.2) (layer "F.Cu") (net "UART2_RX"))
 (segment (start 153.305 84.1925) (end 154 84.8875) (width 0.2) (layer "F.Cu") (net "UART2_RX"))
 (segment (start 154 84.8875) (end 157.675 84.8875) (width 0.2) (layer "F.Cu") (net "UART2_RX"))
 (segment (start 151.35 85.8875) (end 157.675 85.8875) (width 0.2) (layer "F.Cu") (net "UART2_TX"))
 (segment (start 150.765 85.3025) (end 151.35 85.8875) (width 0.2) (layer "F.Cu") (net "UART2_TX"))
 (segment (start 150.765 73.6725) (end 150.765 85.3025) (width 0.2) (layer "F.Cu") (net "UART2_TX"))
 (segment (start 160.68 101.4325) (end 160.68 106.8375) (width 0.2) (layer "F.Cu") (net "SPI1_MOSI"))
 (segment (start 165.575 98.0375) (end 165.575 100.2125) (width 0.2) (layer "F.Cu") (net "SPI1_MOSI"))
 (segment (start 165.225 100.5625) (end 161.55 100.5625) (width 0.2) (layer "F.Cu") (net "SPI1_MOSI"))
 (segment (start 161.55 100.5625) (end 160.68 101.4325) (width 0.2) (layer "F.Cu") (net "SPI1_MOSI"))
 (segment (start 165.575 100.2125) (end 165.225 100.5625) (width 0.2) (layer "F.Cu") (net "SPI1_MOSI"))
 (segment (start 166.575 100.9625) (end 166.575 98.0375) (width 0.2) (layer "F.Cu") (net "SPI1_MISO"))
 (segment (start 165.825 101.7125) (end 166.575 100.9625) (width 0.2) (layer "F.Cu") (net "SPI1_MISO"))
 (segment (start 163.22 102.1925) (end 163.7 101.7125) (width 0.2) (layer "F.Cu") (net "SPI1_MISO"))
 (segment (start 163.7 101.7125) (end 165.825 101.7125) (width 0.2) (layer "F.Cu") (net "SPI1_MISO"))
 (segment (start 163.22 106.8375) (end 163.22 102.1925) (width 0.2) (layer "F.Cu") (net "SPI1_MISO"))
 (segment (start 165.76 102.343186) (end 165.769314 102.343186) (width 0.2) (layer "F.Cu") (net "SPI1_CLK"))
 (segment (start 165.76 106.8375) (end 165.76 102.343186) (width 0.2) (layer "F.Cu") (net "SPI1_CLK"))
 (segment (start 167.575 101.3575) (end 167.575 98.0375) (width 0.2) (layer "F.Cu") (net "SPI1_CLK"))
 (segment (start 167.01 101.9225) (end 167.575 101.3575) (width 0.2) (layer "F.Cu") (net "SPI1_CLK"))
 (segment (start 166.19 101.9225) (end 167.01 101.9225) (width 0.2) (layer "F.Cu") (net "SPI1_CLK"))
 (segment (start 165.769314 102.343186) (end 166.19 101.9225) (width 0.2) (layer "F.Cu") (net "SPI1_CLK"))
 (segment (start 168.575 106.5625) (end 168.3 106.8375) (width 0.2) (layer "F.Cu") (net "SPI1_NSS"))
 (segment (start 168.3 98.3125) (end 168.575 98.0375) (width 0.2) (layer "F.Cu") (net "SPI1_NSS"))
 (segment (start 168.575 98.0375) (end 168.575 106.5625) (width 0.2) (layer "F.Cu") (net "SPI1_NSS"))
 (segment (start 173.71 99.5025) (end 174.28 99.5025) (width 0.2) (layer "F.Cu") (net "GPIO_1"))
 (segment (start 174.405 93.8875) (end 174.53 94.0125) (width 0.2) (layer "F.Cu") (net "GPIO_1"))
 (segment (start 172.475 93.8875) (end 174.405 93.8875) (width 0.2) (layer "F.Cu") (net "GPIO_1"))
 (segment (start 173.38 99.8325) (end 173.71 99.5025) (width 0.2) (layer "F.Cu") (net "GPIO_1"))
 (segment (start 174.53 94.0125) (end 174.53 99.2525) (width 0.2) (layer "F.Cu") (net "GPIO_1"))
 (segment (start 174.28 99.5025) (end 174.53 99.2525) (width 0.2) (layer "F.Cu") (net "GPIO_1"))
 (segment (start 173.38 106.8375) (end 173.38 99.8325) (width 0.2) (layer "F.Cu") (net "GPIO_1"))
 (segment (start 175.125 88.8875) (end 172.475 88.8875) (width 0.2) (layer "F.Cu") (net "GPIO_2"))
 (segment (start 175.92 106.8375) (end 175.92 89.6825) (width 0.2) (layer "F.Cu") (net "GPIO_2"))
 (segment (start 175.92 89.6825) (end 175.125 88.8875) (width 0.2) (layer "F.Cu") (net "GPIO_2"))
 (segment (start 178.46 106.8375) (end 178.485 106.8125) (width 0.2) (layer "F.Cu") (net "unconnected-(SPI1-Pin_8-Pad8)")))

